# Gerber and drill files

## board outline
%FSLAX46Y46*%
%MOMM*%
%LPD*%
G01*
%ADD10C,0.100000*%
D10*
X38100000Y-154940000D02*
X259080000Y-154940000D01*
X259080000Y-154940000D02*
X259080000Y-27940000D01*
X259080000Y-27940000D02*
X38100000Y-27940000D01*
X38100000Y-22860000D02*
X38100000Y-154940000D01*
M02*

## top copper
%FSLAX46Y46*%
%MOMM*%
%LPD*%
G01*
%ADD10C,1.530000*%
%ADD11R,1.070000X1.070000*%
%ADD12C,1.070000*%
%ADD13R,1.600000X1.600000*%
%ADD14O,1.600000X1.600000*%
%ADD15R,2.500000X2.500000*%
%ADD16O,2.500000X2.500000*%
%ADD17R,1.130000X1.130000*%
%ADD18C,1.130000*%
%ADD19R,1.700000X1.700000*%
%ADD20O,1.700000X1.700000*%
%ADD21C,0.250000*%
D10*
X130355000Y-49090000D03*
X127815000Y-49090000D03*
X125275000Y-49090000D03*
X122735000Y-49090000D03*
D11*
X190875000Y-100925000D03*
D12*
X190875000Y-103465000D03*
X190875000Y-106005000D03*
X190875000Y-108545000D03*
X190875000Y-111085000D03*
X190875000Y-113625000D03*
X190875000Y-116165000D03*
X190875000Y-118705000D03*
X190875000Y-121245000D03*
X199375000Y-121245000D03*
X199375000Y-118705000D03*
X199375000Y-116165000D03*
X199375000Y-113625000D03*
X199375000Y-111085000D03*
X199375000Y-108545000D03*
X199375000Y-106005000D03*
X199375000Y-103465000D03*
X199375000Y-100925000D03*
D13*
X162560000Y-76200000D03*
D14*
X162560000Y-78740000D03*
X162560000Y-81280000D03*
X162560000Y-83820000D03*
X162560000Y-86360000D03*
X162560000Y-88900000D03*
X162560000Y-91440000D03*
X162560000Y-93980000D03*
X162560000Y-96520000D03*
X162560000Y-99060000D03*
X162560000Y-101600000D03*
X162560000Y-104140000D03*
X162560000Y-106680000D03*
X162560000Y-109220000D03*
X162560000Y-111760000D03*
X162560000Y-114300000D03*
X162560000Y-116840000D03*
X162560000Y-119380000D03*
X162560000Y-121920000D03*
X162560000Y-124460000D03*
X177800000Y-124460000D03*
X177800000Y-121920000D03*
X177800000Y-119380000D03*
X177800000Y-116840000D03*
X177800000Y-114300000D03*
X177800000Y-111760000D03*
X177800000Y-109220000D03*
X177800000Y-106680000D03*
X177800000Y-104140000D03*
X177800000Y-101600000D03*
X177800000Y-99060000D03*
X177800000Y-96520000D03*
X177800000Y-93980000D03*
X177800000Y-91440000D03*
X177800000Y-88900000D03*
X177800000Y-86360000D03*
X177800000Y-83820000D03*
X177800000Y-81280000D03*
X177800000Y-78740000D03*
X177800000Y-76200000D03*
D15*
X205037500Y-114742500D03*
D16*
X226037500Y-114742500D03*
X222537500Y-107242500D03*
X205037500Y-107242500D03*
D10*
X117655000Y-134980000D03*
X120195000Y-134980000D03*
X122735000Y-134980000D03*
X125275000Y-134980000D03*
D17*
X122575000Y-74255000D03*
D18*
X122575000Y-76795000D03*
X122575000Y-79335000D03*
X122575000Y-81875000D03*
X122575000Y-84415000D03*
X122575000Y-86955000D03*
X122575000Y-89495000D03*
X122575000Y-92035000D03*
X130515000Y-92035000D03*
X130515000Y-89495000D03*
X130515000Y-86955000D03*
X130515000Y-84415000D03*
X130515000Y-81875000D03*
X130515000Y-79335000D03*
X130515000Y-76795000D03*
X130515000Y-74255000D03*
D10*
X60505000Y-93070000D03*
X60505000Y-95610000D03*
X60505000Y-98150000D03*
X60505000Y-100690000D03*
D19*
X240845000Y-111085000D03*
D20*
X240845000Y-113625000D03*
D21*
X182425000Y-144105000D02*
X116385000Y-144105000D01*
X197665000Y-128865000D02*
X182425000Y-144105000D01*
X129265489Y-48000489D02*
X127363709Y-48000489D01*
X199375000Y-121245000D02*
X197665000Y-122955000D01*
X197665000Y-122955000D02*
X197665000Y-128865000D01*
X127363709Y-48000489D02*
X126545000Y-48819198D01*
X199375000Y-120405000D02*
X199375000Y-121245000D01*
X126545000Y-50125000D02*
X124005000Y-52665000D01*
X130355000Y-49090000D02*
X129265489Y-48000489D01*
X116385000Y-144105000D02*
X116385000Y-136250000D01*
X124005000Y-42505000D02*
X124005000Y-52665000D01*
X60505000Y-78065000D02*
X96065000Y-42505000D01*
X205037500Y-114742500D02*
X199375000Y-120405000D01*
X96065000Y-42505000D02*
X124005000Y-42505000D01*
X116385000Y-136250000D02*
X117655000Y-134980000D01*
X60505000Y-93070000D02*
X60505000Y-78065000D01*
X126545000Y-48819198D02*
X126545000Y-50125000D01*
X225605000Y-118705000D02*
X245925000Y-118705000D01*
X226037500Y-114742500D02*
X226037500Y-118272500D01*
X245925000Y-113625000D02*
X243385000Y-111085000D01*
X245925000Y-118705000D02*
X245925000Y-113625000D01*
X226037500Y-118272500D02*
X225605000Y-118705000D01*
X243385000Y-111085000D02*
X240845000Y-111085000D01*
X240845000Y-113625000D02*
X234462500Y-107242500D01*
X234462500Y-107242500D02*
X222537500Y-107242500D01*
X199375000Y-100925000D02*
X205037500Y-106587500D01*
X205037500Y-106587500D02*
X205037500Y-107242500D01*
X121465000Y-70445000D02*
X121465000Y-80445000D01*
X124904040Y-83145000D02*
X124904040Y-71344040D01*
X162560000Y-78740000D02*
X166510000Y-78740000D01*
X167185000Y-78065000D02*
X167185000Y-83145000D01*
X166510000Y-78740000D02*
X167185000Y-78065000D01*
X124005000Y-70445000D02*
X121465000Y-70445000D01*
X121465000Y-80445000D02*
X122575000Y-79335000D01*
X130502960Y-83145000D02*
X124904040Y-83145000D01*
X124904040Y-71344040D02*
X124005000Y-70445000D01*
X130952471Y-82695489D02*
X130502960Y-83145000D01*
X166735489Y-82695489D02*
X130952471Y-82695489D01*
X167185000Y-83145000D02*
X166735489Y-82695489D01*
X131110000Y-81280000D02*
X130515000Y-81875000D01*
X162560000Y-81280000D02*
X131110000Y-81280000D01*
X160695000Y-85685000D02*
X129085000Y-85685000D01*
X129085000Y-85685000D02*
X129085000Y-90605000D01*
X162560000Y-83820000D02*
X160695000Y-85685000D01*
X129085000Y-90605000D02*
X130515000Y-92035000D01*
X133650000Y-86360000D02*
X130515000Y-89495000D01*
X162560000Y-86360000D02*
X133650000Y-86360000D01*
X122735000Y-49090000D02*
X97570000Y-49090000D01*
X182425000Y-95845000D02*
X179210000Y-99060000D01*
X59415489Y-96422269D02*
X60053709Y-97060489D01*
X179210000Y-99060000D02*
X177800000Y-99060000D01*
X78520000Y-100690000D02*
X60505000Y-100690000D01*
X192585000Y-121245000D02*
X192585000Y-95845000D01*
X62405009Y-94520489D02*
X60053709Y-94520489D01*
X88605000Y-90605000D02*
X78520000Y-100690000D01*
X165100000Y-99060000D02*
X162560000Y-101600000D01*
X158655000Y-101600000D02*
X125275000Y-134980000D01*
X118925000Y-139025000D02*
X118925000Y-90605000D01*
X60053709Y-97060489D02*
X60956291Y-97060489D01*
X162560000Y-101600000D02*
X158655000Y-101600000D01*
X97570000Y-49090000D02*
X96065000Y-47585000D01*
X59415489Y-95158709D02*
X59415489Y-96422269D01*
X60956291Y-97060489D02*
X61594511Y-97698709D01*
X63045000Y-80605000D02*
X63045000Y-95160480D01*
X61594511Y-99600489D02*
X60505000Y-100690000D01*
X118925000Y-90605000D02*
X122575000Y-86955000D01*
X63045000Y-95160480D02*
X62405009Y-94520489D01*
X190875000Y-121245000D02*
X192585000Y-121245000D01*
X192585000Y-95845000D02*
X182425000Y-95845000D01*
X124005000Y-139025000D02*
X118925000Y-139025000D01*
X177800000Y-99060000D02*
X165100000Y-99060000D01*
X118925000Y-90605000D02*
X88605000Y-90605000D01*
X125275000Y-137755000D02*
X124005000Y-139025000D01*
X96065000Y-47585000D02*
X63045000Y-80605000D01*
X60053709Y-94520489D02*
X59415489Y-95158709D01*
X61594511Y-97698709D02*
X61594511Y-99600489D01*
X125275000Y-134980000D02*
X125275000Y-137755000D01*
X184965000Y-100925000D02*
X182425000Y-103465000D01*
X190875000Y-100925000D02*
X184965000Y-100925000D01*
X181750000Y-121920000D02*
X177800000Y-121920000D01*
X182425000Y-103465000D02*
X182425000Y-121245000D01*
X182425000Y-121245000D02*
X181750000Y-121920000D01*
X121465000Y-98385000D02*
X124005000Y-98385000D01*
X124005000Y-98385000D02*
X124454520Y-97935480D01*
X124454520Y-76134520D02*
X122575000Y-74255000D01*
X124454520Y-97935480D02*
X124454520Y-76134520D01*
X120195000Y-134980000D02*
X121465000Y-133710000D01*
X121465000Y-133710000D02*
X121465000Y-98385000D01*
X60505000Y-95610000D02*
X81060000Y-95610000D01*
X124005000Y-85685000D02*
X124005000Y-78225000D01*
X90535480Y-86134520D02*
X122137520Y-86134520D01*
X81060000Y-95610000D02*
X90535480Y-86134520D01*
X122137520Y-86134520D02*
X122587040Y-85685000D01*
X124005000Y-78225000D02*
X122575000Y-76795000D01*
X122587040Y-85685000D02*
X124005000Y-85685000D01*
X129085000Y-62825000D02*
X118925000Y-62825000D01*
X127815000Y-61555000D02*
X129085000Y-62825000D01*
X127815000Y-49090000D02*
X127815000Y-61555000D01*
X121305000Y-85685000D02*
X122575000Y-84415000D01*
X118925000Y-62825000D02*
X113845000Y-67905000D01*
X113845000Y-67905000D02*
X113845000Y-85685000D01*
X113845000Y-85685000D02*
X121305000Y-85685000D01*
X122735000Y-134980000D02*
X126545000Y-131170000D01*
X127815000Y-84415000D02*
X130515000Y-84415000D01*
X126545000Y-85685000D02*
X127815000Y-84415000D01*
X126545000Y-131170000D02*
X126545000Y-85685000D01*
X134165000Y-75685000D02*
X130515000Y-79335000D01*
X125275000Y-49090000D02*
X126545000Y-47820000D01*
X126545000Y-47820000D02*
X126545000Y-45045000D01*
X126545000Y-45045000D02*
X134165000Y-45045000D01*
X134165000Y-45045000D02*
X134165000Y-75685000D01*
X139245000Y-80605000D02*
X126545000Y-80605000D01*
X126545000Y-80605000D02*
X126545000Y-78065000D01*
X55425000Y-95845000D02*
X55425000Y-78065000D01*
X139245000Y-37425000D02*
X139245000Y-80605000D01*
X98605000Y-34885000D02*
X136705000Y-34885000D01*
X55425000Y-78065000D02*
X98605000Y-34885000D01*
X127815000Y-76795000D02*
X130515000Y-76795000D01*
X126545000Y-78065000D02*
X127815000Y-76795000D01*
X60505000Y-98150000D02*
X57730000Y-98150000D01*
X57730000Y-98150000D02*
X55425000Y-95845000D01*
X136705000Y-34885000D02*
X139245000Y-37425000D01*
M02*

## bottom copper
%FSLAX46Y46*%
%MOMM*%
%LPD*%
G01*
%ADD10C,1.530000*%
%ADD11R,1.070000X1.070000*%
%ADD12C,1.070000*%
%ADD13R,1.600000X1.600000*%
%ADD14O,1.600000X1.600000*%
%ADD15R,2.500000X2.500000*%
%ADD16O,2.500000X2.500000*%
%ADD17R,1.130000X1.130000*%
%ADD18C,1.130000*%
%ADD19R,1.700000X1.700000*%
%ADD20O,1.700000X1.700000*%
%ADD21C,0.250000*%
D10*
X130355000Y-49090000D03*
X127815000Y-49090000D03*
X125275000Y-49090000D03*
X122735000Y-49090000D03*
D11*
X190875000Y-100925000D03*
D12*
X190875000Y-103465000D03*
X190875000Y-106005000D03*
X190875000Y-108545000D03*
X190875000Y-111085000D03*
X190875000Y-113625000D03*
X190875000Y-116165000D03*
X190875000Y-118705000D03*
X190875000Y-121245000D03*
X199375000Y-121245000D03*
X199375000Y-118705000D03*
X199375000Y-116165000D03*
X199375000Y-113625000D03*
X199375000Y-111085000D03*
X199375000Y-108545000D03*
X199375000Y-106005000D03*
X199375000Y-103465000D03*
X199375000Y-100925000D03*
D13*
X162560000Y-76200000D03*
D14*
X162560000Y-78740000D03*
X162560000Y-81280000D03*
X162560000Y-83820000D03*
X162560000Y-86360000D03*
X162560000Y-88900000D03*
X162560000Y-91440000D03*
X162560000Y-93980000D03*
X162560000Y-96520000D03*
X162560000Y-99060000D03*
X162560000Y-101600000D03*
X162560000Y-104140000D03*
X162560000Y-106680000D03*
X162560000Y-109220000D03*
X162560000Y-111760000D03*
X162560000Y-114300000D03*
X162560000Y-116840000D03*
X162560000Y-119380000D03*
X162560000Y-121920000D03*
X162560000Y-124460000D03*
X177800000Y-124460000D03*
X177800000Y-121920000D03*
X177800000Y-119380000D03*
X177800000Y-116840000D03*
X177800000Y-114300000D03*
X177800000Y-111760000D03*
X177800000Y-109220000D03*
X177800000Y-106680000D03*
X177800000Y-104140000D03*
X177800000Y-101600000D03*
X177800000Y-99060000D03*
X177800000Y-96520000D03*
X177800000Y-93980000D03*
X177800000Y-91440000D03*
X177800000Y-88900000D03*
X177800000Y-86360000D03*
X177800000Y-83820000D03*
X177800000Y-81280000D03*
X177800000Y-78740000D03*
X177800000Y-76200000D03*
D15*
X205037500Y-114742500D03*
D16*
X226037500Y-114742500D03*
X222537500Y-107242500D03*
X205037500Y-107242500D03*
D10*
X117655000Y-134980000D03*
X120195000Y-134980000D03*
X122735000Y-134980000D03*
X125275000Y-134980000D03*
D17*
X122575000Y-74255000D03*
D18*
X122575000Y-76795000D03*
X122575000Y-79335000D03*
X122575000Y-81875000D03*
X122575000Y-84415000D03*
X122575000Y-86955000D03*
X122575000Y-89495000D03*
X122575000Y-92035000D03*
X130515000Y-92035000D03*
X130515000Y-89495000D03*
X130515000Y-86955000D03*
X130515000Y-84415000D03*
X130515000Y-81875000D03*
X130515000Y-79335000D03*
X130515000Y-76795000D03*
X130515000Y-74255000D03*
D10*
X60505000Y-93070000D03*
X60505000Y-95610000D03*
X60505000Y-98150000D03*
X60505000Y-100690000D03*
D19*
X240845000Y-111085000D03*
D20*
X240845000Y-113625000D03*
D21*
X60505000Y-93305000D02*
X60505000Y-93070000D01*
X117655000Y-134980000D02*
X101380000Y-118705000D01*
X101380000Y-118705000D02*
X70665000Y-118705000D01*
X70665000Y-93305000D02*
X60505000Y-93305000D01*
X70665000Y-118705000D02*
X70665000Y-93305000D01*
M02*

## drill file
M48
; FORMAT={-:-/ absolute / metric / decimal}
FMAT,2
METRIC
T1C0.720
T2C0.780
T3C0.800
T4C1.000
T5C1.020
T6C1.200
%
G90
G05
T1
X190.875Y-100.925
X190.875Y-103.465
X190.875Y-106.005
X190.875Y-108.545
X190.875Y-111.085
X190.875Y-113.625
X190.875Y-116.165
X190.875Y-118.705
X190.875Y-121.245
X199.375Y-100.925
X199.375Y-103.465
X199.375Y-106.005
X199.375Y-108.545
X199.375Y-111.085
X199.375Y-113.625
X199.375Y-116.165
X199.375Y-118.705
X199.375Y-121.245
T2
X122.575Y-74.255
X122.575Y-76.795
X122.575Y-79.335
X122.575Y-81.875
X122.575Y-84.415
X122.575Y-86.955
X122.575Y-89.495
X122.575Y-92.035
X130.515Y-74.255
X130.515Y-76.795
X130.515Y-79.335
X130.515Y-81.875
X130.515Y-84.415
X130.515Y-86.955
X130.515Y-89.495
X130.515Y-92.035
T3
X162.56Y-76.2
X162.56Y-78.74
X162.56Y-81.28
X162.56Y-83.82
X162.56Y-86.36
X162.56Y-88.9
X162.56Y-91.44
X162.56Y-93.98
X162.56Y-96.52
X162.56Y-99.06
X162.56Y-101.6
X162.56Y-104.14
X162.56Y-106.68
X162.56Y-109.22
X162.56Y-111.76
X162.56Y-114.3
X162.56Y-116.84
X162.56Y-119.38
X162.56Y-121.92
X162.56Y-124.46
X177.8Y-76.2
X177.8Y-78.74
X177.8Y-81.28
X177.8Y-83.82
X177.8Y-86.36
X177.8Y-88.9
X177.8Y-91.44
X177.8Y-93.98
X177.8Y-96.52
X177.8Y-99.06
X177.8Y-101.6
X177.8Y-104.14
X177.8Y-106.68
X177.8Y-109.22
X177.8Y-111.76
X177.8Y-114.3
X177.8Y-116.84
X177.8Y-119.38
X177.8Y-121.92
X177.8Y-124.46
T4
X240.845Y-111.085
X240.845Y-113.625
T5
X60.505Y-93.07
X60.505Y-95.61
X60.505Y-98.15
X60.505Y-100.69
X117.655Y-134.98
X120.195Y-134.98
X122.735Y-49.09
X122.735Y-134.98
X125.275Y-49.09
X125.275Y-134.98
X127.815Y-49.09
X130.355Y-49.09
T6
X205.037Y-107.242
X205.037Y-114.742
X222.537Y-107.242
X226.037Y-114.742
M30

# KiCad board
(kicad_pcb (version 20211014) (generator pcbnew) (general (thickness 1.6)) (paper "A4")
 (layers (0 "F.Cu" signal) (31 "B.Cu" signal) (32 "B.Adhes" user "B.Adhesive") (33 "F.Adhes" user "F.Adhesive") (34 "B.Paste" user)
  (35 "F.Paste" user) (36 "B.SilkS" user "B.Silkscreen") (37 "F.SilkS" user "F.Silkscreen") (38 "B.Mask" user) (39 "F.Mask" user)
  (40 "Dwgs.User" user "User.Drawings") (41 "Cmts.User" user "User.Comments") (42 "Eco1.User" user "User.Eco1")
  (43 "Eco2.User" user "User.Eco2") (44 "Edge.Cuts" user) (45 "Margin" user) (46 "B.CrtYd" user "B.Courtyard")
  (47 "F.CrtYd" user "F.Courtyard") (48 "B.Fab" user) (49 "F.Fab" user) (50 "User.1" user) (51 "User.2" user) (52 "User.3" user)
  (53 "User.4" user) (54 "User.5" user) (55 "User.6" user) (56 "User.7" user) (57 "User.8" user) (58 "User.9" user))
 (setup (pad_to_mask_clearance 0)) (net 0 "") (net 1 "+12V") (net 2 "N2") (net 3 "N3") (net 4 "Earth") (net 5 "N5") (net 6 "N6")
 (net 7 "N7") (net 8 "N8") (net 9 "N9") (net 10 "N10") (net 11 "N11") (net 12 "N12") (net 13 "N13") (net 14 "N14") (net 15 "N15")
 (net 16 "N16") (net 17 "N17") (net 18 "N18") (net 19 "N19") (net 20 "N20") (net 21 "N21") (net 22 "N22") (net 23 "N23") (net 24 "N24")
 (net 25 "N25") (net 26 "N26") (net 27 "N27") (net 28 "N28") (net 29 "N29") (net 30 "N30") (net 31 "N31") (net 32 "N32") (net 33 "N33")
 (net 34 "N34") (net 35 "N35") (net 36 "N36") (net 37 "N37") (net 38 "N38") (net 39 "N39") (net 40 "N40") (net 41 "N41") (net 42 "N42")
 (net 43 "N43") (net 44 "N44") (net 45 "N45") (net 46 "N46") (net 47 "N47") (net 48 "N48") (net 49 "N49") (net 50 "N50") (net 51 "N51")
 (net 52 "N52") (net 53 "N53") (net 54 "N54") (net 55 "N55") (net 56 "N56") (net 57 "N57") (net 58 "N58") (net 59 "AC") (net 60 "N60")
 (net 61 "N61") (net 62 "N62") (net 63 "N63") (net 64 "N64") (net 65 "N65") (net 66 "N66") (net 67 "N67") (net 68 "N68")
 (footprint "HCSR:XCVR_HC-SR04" (layer "F.Cu") (at 126.545 49.09 180)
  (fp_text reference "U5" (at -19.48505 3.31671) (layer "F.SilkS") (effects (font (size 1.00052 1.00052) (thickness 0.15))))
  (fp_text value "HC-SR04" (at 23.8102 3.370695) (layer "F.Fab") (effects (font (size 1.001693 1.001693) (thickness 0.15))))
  (pad "1" thru_hole circle locked (at -3.81 0 180) (size 1.53 1.53) (drill 1.02) (layers *.Cu *.Mask) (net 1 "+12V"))
  (pad "2" thru_hole circle locked (at -1.27 0 180) (size 1.53 1.53) (drill 1.02) (layers *.Cu *.Mask) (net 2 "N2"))
  (pad "3" thru_hole circle locked (at 1.27 0 180) (size 1.53 1.53) (drill 1.02) (layers *.Cu *.Mask) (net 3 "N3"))
  (pad "4" thru_hole circle locked (at 3.81 0 180) (size 1.53 1.53) (drill 1.02) (layers *.Cu *.Mask) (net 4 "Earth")))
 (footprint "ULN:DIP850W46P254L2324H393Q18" (layer "F.Cu") (at 195.125 111.085)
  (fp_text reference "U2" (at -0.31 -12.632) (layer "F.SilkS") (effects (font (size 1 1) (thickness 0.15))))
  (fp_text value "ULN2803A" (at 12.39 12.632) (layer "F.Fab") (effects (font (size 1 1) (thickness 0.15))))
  (pad "1" thru_hole rect locked (at -4.25 -10.16) (size 1.07 1.07) (drill 0.72) (layers *.Cu *.Mask) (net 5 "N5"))
  (pad "2" thru_hole circle locked (at -4.25 -7.62) (size 1.07 1.07) (drill 0.72) (layers *.Cu *.Mask) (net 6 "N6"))
  (pad "3" thru_hole circle locked (at -4.25 -5.08) (size 1.07 1.07) (drill 0.72) (layers *.Cu *.Mask) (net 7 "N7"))
  (pad "4" thru_hole circle locked (at -4.25 -2.54) (size 1.07 1.07) (drill 0.72) (layers *.Cu *.Mask) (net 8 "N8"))
  (pad "5" thru_hole circle locked (at -4.25 0) (size 1.07 1.07) (drill 0.72) (layers *.Cu *.Mask) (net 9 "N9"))
  (pad "6" thru_hole circle locked (at -4.25 2.54) (size 1.07 1.07) (drill 0.72) (layers *.Cu *.Mask) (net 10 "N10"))
  (pad "7" thru_hole circle locked (at -4.25 5.08) (size 1.07 1.07) (drill 0.72) (layers *.Cu *.Mask) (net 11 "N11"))
  (pad "8" thru_hole circle locked (at -4.25 7.62) (size 1.07 1.07) (drill 0.72) (layers *.Cu *.Mask) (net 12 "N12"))
  (pad "9" thru_hole circle locked (at -4.25 10.16) (size 1.07 1.07) (drill 0.72) (layers *.Cu *.Mask) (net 4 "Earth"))
  (pad "10" thru_hole circle locked (at 4.25 10.16) (size 1.07 1.07) (drill 0.72) (layers *.Cu *.Mask) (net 1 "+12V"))
  (pad "11" thru_hole circle locked (at 4.25 7.62) (size 1.07 1.07) (drill 0.72) (layers *.Cu *.Mask) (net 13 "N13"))
  (pad "12" thru_hole circle locked (at 4.25 5.08) (size 1.07 1.07) (drill 0.72) (layers *.Cu *.Mask) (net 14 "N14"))
  (pad "13" thru_hole circle locked (at 4.25 2.54) (size 1.07 1.07) (drill 0.72) (layers *.Cu *.Mask) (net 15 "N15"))
  (pad "14" thru_hole circle locked (at 4.25 0) (size 1.07 1.07) (drill 0.72) (layers *.Cu *.Mask) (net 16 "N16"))
  (pad "15" thru_hole circle locked (at 4.25 -2.54) (size 1.07 1.07) (drill 0.72) (layers *.Cu *.Mask) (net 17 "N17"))
  (pad "16" thru_hole circle locked (at 4.25 -5.08) (size 1.07 1.07) (drill 0.72) (layers *.Cu *.Mask) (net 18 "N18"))
  (pad "17" thru_hole circle locked (at 4.25 -7.62) (size 1.07 1.07) (drill 0.72) (layers *.Cu *.Mask) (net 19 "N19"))
  (pad "18" thru_hole circle locked (at 4.25 -10.16) (size 1.07 1.07) (drill 0.72) (layers *.Cu *.Mask) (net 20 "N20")))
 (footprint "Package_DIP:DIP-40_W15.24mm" (layer "F.Cu") (at 162.56 76.2)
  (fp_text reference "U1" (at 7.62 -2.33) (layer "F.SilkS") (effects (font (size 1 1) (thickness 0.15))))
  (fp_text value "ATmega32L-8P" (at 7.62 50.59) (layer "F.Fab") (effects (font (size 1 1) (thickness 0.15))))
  (pad "1" thru_hole rect (at 0 0) (size 1.6 1.6) (drill 0.8) (layers *.Cu *.Mask) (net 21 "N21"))
  (pad "2" thru_hole oval (at 0 2.54) (size 1.6 1.6) (drill 0.8) (layers *.Cu *.Mask) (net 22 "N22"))
  (pad "3" thru_hole oval (at 0 5.08) (size 1.6 1.6) (drill 0.8) (layers *.Cu *.Mask) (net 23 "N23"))
  (pad "4" thru_hole oval (at 0 7.62) (size 1.6 1.6) (drill 0.8) (layers *.Cu *.Mask) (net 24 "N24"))
  (pad "5" thru_hole oval (at 0 10.16) (size 1.6 1.6) (drill 0.8) (layers *.Cu *.Mask) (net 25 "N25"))
  (pad "6" thru_hole oval (at 0 12.7) (size 1.6 1.6) (drill 0.8) (layers *.Cu *.Mask) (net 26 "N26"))
  (pad "7" thru_hole oval (at 0 15.24) (size 1.6 1.6) (drill 0.8) (layers *.Cu *.Mask) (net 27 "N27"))
  (pad "8" thru_hole oval (at 0 17.78) (size 1.6 1.6) (drill 0.8) (layers *.Cu *.Mask) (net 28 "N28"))
  (pad "9" thru_hole oval (at 0 20.32) (size 1.6 1.6) (drill 0.8) (layers *.Cu *.Mask) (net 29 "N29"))
  (pad "10" thru_hole oval (at 0 22.86) (size 1.6 1.6) (drill 0.8) (layers *.Cu *.Mask) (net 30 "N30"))
  (pad "11" thru_hole oval (at 0 25.4) (size 1.6 1.6) (drill 0.8) (layers *.Cu *.Mask) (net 4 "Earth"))
  (pad "12" thru_hole oval (at 0 27.94) (size 1.6 1.6) (drill 0.8) (layers *.Cu *.Mask) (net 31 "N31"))
  (pad "13" thru_hole oval (at 0 30.48) (size 1.6 1.6) (drill 0.8) (layers *.Cu *.Mask) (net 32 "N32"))
  (pad "14" thru_hole oval (at 0 33.02) (size 1.6 1.6) (drill 0.8) (layers *.Cu *.Mask) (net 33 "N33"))
  (pad "15" thru_hole oval (at 0 35.56) (size 1.6 1.6) (drill 0.8) (layers *.Cu *.Mask) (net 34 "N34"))
  (pad "16" thru_hole oval (at 0 38.1) (size 1.6 1.6) (drill 0.8) (layers *.Cu *.Mask) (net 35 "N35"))
  (pad "17" thru_hole oval (at 0 40.64) (size 1.6 1.6) (drill 0.8) (layers *.Cu *.Mask) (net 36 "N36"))
  (pad "18" thru_hole oval (at 0 43.18) (size 1.6 1.6) (drill 0.8) (layers *.Cu *.Mask) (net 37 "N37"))
  (pad "19" thru_hole oval (at 0 45.72) (size 1.6 1.6) (drill 0.8) (layers *.Cu *.Mask) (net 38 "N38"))
  (pad "20" thru_hole oval (at 0 48.26) (size 1.6 1.6) (drill 0.8) (layers *.Cu *.Mask) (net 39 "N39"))
  (pad "21" thru_hole oval (at 15.24 48.26) (size 1.6 1.6) (drill 0.8) (layers *.Cu *.Mask) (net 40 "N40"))
  (pad "22" thru_hole oval (at 15.24 45.72) (size 1.6 1.6) (drill 0.8) (layers *.Cu *.Mask) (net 5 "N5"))
  (pad "23" thru_hole oval (at 15.24 43.18) (size 1.6 1.6) (drill 0.8) (layers *.Cu *.Mask) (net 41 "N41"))
  (pad "24" thru_hole oval (at 15.24 40.64) (size 1.6 1.6) (drill 0.8) (layers *.Cu *.Mask) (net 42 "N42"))
  (pad "25" thru_hole oval (at 15.24 38.1) (size 1.6 1.6) (drill 0.8) (layers *.Cu *.Mask) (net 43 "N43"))
  (pad "26" thru_hole oval (at 15.24 35.56) (size 1.6 1.6) (drill 0.8) (layers *.Cu *.Mask) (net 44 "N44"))
  (pad "27" thru_hole oval (at 15.24 33.02) (size 1.6 1.6) (drill 0.8) (layers *.Cu *.Mask) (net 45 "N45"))
  (pad "28" thru_hole oval (at 15.24 30.48) (size 1.6 1.6) (drill 0.8) (layers *.Cu *.Mask) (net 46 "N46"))
  (pad "29" thru_hole oval (at 15.24 27.94) (size 1.6 1.6) (drill 0.8) (layers *.Cu *.Mask) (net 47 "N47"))
  (pad "30" thru_hole oval (at 15.24 25.4) (size 1.6 1.6) (drill 0.8) (layers *.Cu *.Mask) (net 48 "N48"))
  (pad "31" thru_hole oval (at 15.24 22.86) (size 1.6 1.6) (drill 0.8) (layers *.Cu *.Mask) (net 4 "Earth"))
  (pad "32" thru_hole oval (at 15.24 20.32) (size 1.6 1.6) (drill 0.8) (layers *.Cu *.Mask) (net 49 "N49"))
  (pad "33" thru_hole oval (at 15.24 17.78) (size 1.6 1.6) (drill 0.8) (layers *.Cu *.Mask) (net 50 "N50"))
  (pad "34" thru_hole oval (at 15.24 15.24) (size 1.6 1.6) (drill 0.8) (layers *.Cu *.Mask) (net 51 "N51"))
  (pad "35" thru_hole oval (at 15.24 12.7) (size 1.6 1.6) (drill 0.8) (layers *.Cu *.Mask) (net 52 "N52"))
  (pad "36" thru_hole oval (at 15.24 10.16) (size 1.6 1.6) (drill 0.8) (layers *.Cu *.Mask) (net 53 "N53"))
  (pad "37" thru_hole oval (at 15.24 7.62) (size 1.6 1.6) (drill 0.8) (layers *.Cu *.Mask) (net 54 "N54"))
  (pad "38" thru_hole oval (at 15.24 5.08) (size 1.6 1.6) (drill 0.8) (layers *.Cu *.Mask) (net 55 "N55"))
  (pad "39" thru_hole oval (at 15.24 2.54) (size 1.6 1.6) (drill 0.8) (layers *.Cu *.Mask) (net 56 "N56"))
  (pad "40" thru_hole oval (at 15.24 0) (size 1.6 1.6) (drill 0.8) (layers *.Cu *.Mask) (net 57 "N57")))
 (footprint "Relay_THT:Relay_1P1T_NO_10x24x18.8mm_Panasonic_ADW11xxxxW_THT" (layer "F.Cu") (at 205.0375 114.7425 90)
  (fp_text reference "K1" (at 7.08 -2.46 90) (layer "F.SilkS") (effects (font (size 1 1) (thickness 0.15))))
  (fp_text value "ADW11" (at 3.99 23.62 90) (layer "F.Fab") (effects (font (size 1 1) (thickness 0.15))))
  (pad "1" thru_hole rect (at 0 0 90) (size 2.5 2.5) (drill 1.2) (layers *.Cu *.Mask) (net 1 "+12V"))
  (pad "3" thru_hole oval (at 0 21 90) (size 2.5 2.5) (drill 1.2) (layers *.Cu *.Mask) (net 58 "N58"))
  (pad "5" thru_hole oval (at 7.5 17.5 90) (size 2.5 2.5) (drill 1.2) (layers *.Cu *.Mask) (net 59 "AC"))
  (pad "6" thru_hole oval (at 7.5 0 90) (size 2.5 2.5) (drill 1.2) (layers *.Cu *.Mask) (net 20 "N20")))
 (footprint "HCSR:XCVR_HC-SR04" (layer "F.Cu") (at 121.465 134.98)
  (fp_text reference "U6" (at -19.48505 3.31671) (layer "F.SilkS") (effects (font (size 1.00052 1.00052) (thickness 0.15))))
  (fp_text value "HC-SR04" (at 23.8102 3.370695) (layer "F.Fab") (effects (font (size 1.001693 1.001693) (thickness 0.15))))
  (pad "1" thru_hole circle locked (at -3.81 0) (size 1.53 1.53) (drill 1.02) (layers *.Cu *.Mask) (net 1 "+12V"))
  (pad "2" thru_hole circle locked (at -1.27 0) (size 1.53 1.53) (drill 1.02) (layers *.Cu *.Mask) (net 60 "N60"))
  (pad "3" thru_hole circle locked (at 1.27 0) (size 1.53 1.53) (drill 1.02) (layers *.Cu *.Mask) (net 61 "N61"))
  (pad "4" thru_hole circle locked (at 3.81 0) (size 1.53 1.53) (drill 1.02) (layers *.Cu *.Mask) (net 4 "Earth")))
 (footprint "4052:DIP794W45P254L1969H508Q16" (layer "F.Cu") (at 126.545 83.145)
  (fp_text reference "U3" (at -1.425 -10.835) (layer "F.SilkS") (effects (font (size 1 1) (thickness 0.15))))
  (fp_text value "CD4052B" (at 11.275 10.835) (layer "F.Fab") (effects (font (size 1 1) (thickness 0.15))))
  (pad "1" thru_hole rect locked (at -3.97 -8.89) (size 1.13 1.13) (drill 0.78) (layers *.Cu *.Mask) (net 60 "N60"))
  (pad "2" thru_hole circle locked (at -3.97 -6.35) (size 1.13 1.13) (drill 0.78) (layers *.Cu *.Mask) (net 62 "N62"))
  (pad "3" thru_hole circle locked (at -3.97 -3.81) (size 1.13 1.13) (drill 0.78) (layers *.Cu *.Mask) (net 22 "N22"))
  (pad "4" thru_hole circle locked (at -3.97 -1.27) (size 1.13 1.13) (drill 0.78) (layers *.Cu *.Mask) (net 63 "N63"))
  (pad "5" thru_hole circle locked (at -3.97 1.27) (size 1.13 1.13) (drill 0.78) (layers *.Cu *.Mask) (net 2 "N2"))
  (pad "6" thru_hole circle locked (at -3.97 3.81) (size 1.13 1.13) (drill 0.78) (layers *.Cu *.Mask) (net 4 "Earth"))
  (pad "7" thru_hole circle locked (at -3.97 6.35) (size 1.13 1.13) (drill 0.78) (layers *.Cu *.Mask) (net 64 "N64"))
  (pad "8" thru_hole circle locked (at -3.97 8.89) (size 1.13 1.13) (drill 0.78) (layers *.Cu *.Mask) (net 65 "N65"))
  (pad "9" thru_hole circle locked (at 3.97 8.89) (size 1.13 1.13) (drill 0.78) (layers *.Cu *.Mask) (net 24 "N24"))
  (pad "10" thru_hole circle locked (at 3.97 6.35) (size 1.13 1.13) (drill 0.78) (layers *.Cu *.Mask) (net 25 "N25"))
  (pad "11" thru_hole circle locked (at 3.97 3.81) (size 1.13 1.13) (drill 0.78) (layers *.Cu *.Mask) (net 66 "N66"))
  (pad "12" thru_hole circle locked (at 3.97 1.27) (size 1.13 1.13) (drill 0.78) (layers *.Cu *.Mask) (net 61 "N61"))
  (pad "13" thru_hole circle locked (at 3.97 -1.27) (size 1.13 1.13) (drill 0.78) (layers *.Cu *.Mask) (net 23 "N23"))
  (pad "14" thru_hole circle locked (at 3.97 -3.81) (size 1.13 1.13) (drill 0.78) (layers *.Cu *.Mask) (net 3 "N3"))
  (pad "15" thru_hole circle locked (at 3.97 -6.35) (size 1.13 1.13) (drill 0.78) (layers *.Cu *.Mask) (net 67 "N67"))
  (pad "16" thru_hole circle locked (at 3.97 -8.89) (size 1.13 1.13) (drill 0.78) (layers *.Cu *.Mask) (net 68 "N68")))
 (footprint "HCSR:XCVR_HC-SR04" (layer "F.Cu") (at 60.505 96.88 -90)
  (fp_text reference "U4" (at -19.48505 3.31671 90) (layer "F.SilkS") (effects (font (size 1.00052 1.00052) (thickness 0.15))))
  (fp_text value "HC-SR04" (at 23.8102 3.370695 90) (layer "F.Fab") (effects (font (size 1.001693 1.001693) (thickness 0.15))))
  (pad "1" thru_hole circle locked (at -3.81 0 270) (size 1.53 1.53) (drill 1.02) (layers *.Cu *.Mask) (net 1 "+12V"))
  (pad "2" thru_hole circle locked (at -1.27 0 270) (size 1.53 1.53) (drill 1.02) (layers *.Cu *.Mask) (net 62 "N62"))
  (pad "3" thru_hole circle locked (at 1.27 0 270) (size 1.53 1.53) (drill 1.02) (layers *.Cu *.Mask) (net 67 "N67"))
  (pad "4" thru_hole circle locked (at 3.81 0 270) (size 1.53 1.53) (drill 1.02) (layers *.Cu *.Mask) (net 4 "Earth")))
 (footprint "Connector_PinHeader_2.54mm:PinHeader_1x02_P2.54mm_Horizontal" (layer "F.Cu") (at 240.845 111.085)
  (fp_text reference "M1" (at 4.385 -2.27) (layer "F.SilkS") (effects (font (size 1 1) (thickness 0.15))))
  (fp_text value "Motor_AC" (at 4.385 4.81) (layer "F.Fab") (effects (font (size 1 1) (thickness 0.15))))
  (pad "1" thru_hole rect (at 0 0) (size 1.7 1.7) (drill 1) (layers *.Cu *.Mask) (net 58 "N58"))
  (pad "2" thru_hole oval (at 0 2.54) (size 1.7 1.7) (drill 1) (layers *.Cu *.Mask) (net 59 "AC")))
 (gr_line (start 38.1 154.94) (end 259.08 154.94) (layer "Edge.Cuts") (width 0.1))
 (gr_line (start 259.08 154.94) (end 259.08 27.94) (layer "Edge.Cuts") (width 0.1))
 (gr_line (start 259.08 27.94) (end 38.1 27.94) (layer "Edge.Cuts") (width 0.1))
 (gr_line (start 38.1 22.86) (end 38.1 154.94) (layer "Edge.Cuts") (width 0.1))
 (segment (start 182.425 144.105) (end 116.385 144.105) (width 0.25) (layer "F.Cu") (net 1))
 (segment (start 197.665 128.865) (end 182.425 144.105) (width 0.25) (layer "F.Cu") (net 1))
 (segment (start 129.265489 48.000489) (end 127.363709 48.000489) (width 0.25) (layer "F.Cu") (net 1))
 (segment (start 199.375 121.245) (end 197.665 122.955) (width 0.25) (layer "F.Cu") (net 1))
 (segment (start 197.665 122.955) (end 197.665 128.865) (width 0.25) (layer "F.Cu") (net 1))
 (segment (start 127.363709 48.000489) (end 126.545 48.819198) (width 0.25) (layer "F.Cu") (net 1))
 (segment (start 199.375 120.405) (end 199.375 121.245) (width 0.25) (layer "F.Cu") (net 1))
 (segment (start 126.545 50.125) (end 124.005 52.665) (width 0.25) (layer "F.Cu") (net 1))
 (segment (start 130.355 49.09) (end 129.265489 48.000489) (width 0.25) (layer "F.Cu") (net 1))
 (segment (start 116.385 144.105) (end 116.385 136.25) (width 0.25) (layer "F.Cu") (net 1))
 (segment (start 124.005 42.505) (end 124.005 52.665) (width 0.25) (layer "F.Cu") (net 1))
 (segment (start 60.505 78.065) (end 96.065 42.505) (width 0.25) (layer "F.Cu") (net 1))
 (segment (start 205.0375 114.7425) (end 199.375 120.405) (width 0.25) (layer "F.Cu") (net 1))
 (segment (start 96.065 42.505) (end 124.005 42.505) (width 0.25) (layer "F.Cu") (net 1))
 (segment (start 116.385 136.25) (end 117.655 134.98) (width 0.25) (layer "F.Cu") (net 1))
 (segment (start 60.505 93.07) (end 60.505 78.065) (width 0.25) (layer "F.Cu") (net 1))
 (segment (start 126.545 48.819198) (end 126.545 50.125) (width 0.25) (layer "F.Cu") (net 1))
 (segment (start 60.505 93.305) (end 60.505 93.07) (width 0.25) (layer "B.Cu") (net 1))
 (segment (start 117.655 134.98) (end 101.38 118.705) (width 0.25) (layer "B.Cu") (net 1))
 (segment (start 101.38 118.705) (end 70.665 118.705) (width 0.25) (layer "B.Cu") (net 1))
 (segment (start 70.665 93.305) (end 60.505 93.305) (width 0.25) (layer "B.Cu") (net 1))
 (segment (start 70.665 118.705) (end 70.665 93.305) (width 0.25) (layer "B.Cu") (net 1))
 (segment (start 225.605 118.705) (end 245.925 118.705) (width 0.25) (layer "F.Cu") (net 58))
 (segment (start 226.0375 114.7425) (end 226.0375 118.2725) (width 0.25) (layer "F.Cu") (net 58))
 (segment (start 245.925 113.625) (end 243.385 111.085) (width 0.25) (layer "F.Cu") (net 58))
 (segment (start 245.925 118.705) (end 245.925 113.625) (width 0.25) (layer "F.Cu") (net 58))
 (segment (start 226.0375 118.2725) (end 225.605 118.705) (width 0.25) (layer "F.Cu") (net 58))
 (segment (start 243.385 111.085) (end 240.845 111.085) (width 0.25) (layer "F.Cu") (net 58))
 (segment (start 240.845 113.625) (end 234.4625 107.2425) (width 0.25) (layer "F.Cu") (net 59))
 (segment (start 234.4625 107.2425) (end 222.5375 107.2425) (width 0.25) (layer "F.Cu") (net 59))
 (segment (start 199.375 100.925) (end 205.0375 106.5875) (width 0.25) (layer "F.Cu") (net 20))
 (segment (start 205.0375 106.5875) (end 205.0375 107.2425) (width 0.25) (layer "F.Cu") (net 20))
 (segment (start 121.465 70.445) (end 121.465 80.445) (width 0.25) (layer "F.Cu") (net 22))
 (segment (start 124.90404 83.145) (end 124.90404 71.34404) (width 0.25) (layer "F.Cu") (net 22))
 (segment (start 162.56 78.74) (end 166.51 78.74) (width 0.25) (layer "F.Cu") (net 22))
 (segment (start 167.185 78.065) (end 167.185 83.145) (width 0.25) (layer "F.Cu") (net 22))
 (segment (start 166.51 78.74) (end 167.185 78.065) (width 0.25) (layer "F.Cu") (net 22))
 (segment (start 124.005 70.445) (end 121.465 70.445) (width 0.25) (layer "F.Cu") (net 22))
 (segment (start 121.465 80.445) (end 122.575 79.335) (width 0.25) (layer "F.Cu") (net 22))
 (segment (start 130.50296 83.145) (end 124.90404 83.145) (width 0.25) (layer "F.Cu") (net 22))
 (segment (start 124.90404 71.34404) (end 124.005 70.445) (width 0.25) (layer "F.Cu") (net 22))
 (segment (start 130.952471 82.695489) (end 130.50296 83.145) (width 0.25) (layer "F.Cu") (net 22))
 (segment (start 166.735489 82.695489) (end 130.952471 82.695489) (width 0.25) (layer "F.Cu") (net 22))
 (segment (start 167.185 83.145) (end 166.735489 82.695489) (width 0.25) (layer "F.Cu") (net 22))
 (segment (start 131.11 81.28) (end 130.515 81.875) (width 0.25) (layer "F.Cu") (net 23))
 (segment (start 162.56 81.28) (end 131.11 81.28) (width 0.25) (layer "F.Cu") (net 23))
 (segment (start 160.695 85.685) (end 129.085 85.685) (width 0.25) (layer "F.Cu") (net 24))
 (segment (start 129.085 85.685) (end 129.085 90.605) (width 0.25) (layer "F.Cu") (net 24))
 (segment (start 162.56 83.82) (end 160.695 85.685) (width 0.25) (layer "F.Cu") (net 24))
 (segment (start 129.085 90.605) (end 130.515 92.035) (width 0.25) (layer "F.Cu") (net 24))
 (segment (start 133.65 86.36) (end 130.515 89.495) (width 0.25) (layer "F.Cu") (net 25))
 (segment (start 162.56 86.36) (end 133.65 86.36) (width 0.25) (layer "F.Cu") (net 25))
 (segment (start 122.735 49.09) (end 97.57 49.09) (width 0.25) (layer "F.Cu") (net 4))
 (segment (start 182.425 95.845) (end 179.21 99.06) (width 0.25) (layer "F.Cu") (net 4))
 (segment (start 59.415489 96.422269) (end 60.053709 97.060489) (width 0.25) (layer "F.Cu") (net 4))
 (segment (start 179.21 99.06) (end 177.8 99.06) (width 0.25) (layer "F.Cu") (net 4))
 (segment (start 78.52 100.69) (end 60.505 100.69) (width 0.25) (layer "F.Cu") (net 4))
 (segment (start 192.585 121.245) (end 192.585 95.845) (width 0.25) (layer "F.Cu") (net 4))
 (segment (start 62.405009 94.520489) (end 60.053709 94.520489) (width 0.25) (layer "F.Cu") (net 4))
 (segment (start 88.605 90.605) (end 78.52 100.69) (width 0.25) (layer "F.Cu") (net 4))
 (segment (start 165.1 99.06) (end 162.56 101.6) (width 0.25) (layer "F.Cu") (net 4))
 (segment (start 158.655 101.6) (end 125.275 134.98) (width 0.25) (layer "F.Cu") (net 4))
 (segment (start 118.925 139.025) (end 118.925 90.605) (width 0.25) (layer "F.Cu") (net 4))
 (segment (start 60.053709 97.060489) (end 60.956291 97.060489) (width 0.25) (layer "F.Cu") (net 4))
 (segment (start 162.56 101.6) (end 158.655 101.6) (width 0.25) (layer "F.Cu") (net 4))
 (segment (start 97.57 49.09) (end 96.065 47.585) (width 0.25) (layer "F.Cu") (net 4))
 (segment (start 59.415489 95.158709) (end 59.415489 96.422269) (width 0.25) (layer "F.Cu") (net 4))
 (segment (start 60.956291 97.060489) (end 61.594511 97.698709) (width 0.25) (layer "F.Cu") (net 4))
 (segment (start 63.045 80.605) (end 63.045 95.16048) (width 0.25) (layer "F.Cu") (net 4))
 (segment (start 61.594511 99.600489) (end 60.505 100.69) (width 0.25) (layer "F.Cu") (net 4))
 (segment (start 118.925 90.605) (end 122.575 86.955) (width 0.25) (layer "F.Cu") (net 4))
 (segment (start 63.045 95.16048) (end 62.405009 94.520489) (width 0.25) (layer "F.Cu") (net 4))
 (segment (start 190.875 121.245) (end 192.585 121.245) (width 0.25) (layer "F.Cu") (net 4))
 (segment (start 192.585 95.845) (end 182.425 95.845) (width 0.25) (layer "F.Cu") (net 4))
 (segment (start 124.005 139.025) (end 118.925 139.025) (width 0.25) (layer "F.Cu") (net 4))
 (segment (start 177.8 99.06) (end 165.1 99.06) (width 0.25) (layer "F.Cu") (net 4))
 (segment (start 118.925 90.605) (end 88.605 90.605) (width 0.25) (layer "F.Cu") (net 4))
 (segment (start 125.275 137.755) (end 124.005 139.025) (width 0.25) (layer "F.Cu") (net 4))
 (segment (start 96.065 47.585) (end 63.045 80.605) (width 0.25) (layer "F.Cu") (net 4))
 (segment (start 60.053709 94.520489) (end 59.415489 95.158709) (width 0.25) (layer "F.Cu") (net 4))
 (segment (start 61.594511 97.698709) (end 61.594511 99.600489) (width 0.25) (layer "F.Cu") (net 4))
 (segment (start 125.275 134.98) (end 125.275 137.755) (width 0.25) (layer "F.Cu") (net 4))
 (segment (start 184.965 100.925) (end 182.425 103.465) (width 0.25) (layer "F.Cu") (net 5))
 (segment (start 190.875 100.925) (end 184.965 100.925) (width 0.25) (layer "F.Cu") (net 5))
 (segment (start 181.75 121.92) (end 177.8 121.92) (width 0.25) (layer "F.Cu") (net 5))
 (segment (start 182.425 103.465) (end 182.425 121.245) (width 0.25) (layer "F.Cu") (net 5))
 (segment (start 182.425 121.245) (end 181.75 121.92) (width 0.25) (layer "F.Cu") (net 5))
 (segment (start 121.465 98.385) (end 124.005 98.385) (width 0.25) (layer "F.Cu") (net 60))
 (segment (start 124.005 98.385) (end 124.45452 97.93548) (width 0.25) (layer "F.Cu") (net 60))
 (segment (start 124.45452 76.13452) (end 122.575 74.255) (width 0.25) (layer "F.Cu") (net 60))
 (segment (start 124.45452 97.93548) (end 124.45452 76.13452) (width 0.25) (layer "F.Cu") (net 60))
 (segment (start 120.195 134.98) (end 121.465 133.71) (width 0.25) (layer "F.Cu") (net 60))
 (segment (start 121.465 133.71) (end 121.465 98.385) (width 0.25) (layer "F.Cu") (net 60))
 (segment (start 60.505 95.61) (end 81.06 95.61) (width 0.25) (layer "F.Cu") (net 62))
 (segment (start 124.005 85.685) (end 124.005 78.225) (width 0.25) (layer "F.Cu") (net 62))
 (segment (start 90.53548 86.13452) (end 122.13752 86.13452) (width 0.25) (layer "F.Cu") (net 62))
 (segment (start 81.06 95.61) (end 90.53548 86.13452) (width 0.25) (layer "F.Cu") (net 62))
 (segment (start 122.13752 86.13452) (end 122.58704 85.685) (width 0.25) (layer "F.Cu") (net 62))
 (segment (start 124.005 78.225) (end 122.575 76.795) (width 0.25) (layer "F.Cu") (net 62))
 (segment (start 122.58704 85.685) (end 124.005 85.685) (width 0.25) (layer "F.Cu") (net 62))
 (segment (start 129.085 62.825) (end 118.925 62.825) (width 0.25) (layer "F.Cu") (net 2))
 (segment (start 127.815 61.555) (end 129.085 62.825) (width 0.25) (layer "F.Cu") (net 2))
 (segment (start 127.815 49.09) (end 127.815 61.555) (width 0.25) (layer "F.Cu") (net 2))
 (segment (start 121.305 85.685) (end 122.575 84.415) (width 0.25) (layer "F.Cu") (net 2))
 (segment (start 118.925 62.825) (end 113.845 67.905) (width 0.25) (layer "F.Cu") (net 2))
 (segment (start 113.845 67.905) (end 113.845 85.685) (width 0.25) (layer "F.Cu") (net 2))
 (segment (start 113.845 85.685) (end 121.305 85.685) (width 0.25) (layer "F.Cu") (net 2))
 (segment (start 122.735 134.98) (end 126.545 131.17) (width 0.25) (layer "F.Cu") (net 61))
 (segment (start 127.815 84.415) (end 130.515 84.415) (width 0.25) (layer "F.Cu") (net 61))
 (segment (start 126.545 85.685) (end 127.815 84.415) (width 0.25) (layer "F.Cu") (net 61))
 (segment (start 126.545 131.17) (end 126.545 85.685) (width 0.25) (layer "F.Cu") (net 61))
 (segment (start 134.165 75.685) (end 130.515 79.335) (width 0.25) (layer "F.Cu") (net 3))
 (segment (start 125.275 49.09) (end 126.545 47.82) (width 0.25) (layer "F.Cu") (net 3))
 (segment (start 126.545 47.82) (end 126.545 45.045) (width 0.25) (layer "F.Cu") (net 3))
 (segment (start 126.545 45.045) (end 134.165 45.045) (width 0.25) (layer "F.Cu") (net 3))
 (segment (start 134.165 45.045) (end 134.165 75.685) (width 0.25) (layer "F.Cu") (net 3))
 (segment (start 139.245 80.605) (end 126.545 80.605) (width 0.25) (layer "F.Cu") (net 67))
 (segment (start 126.545 80.605) (end 126.545 78.065) (width 0.25) (layer "F.Cu") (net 67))
 (segment (start 55.425 95.845) (end 55.425 78.065) (width 0.25) (layer "F.Cu") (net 67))
 (segment (start 139.245 37.425) (end 139.245 80.605) (width 0.25) (layer "F.Cu") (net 67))
 (segment (start 98.605 34.885) (end 136.705 34.885) (width 0.25) (layer "F.Cu") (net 67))
 (segment (start 55.425 78.065) (end 98.605 34.885) (width 0.25) (layer "F.Cu") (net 67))
 (segment (start 127.815 76.795) (end 130.515 76.795) (width 0.25) (layer "F.Cu") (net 67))
 (segment (start 126.545 78.065) (end 127.815 76.795) (width 0.25) (layer "F.Cu") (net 67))
 (segment (start 60.505 98.15) (end 57.73 98.15) (width 0.25) (layer "F.Cu") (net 67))
 (segment (start 57.73 98.15) (end 55.425 95.845) (width 0.25) (layer "F.Cu") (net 67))
 (segment (start 136.705 34.885) (end 139.245 37.425) (width 0.25) (layer "F.Cu") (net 67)))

